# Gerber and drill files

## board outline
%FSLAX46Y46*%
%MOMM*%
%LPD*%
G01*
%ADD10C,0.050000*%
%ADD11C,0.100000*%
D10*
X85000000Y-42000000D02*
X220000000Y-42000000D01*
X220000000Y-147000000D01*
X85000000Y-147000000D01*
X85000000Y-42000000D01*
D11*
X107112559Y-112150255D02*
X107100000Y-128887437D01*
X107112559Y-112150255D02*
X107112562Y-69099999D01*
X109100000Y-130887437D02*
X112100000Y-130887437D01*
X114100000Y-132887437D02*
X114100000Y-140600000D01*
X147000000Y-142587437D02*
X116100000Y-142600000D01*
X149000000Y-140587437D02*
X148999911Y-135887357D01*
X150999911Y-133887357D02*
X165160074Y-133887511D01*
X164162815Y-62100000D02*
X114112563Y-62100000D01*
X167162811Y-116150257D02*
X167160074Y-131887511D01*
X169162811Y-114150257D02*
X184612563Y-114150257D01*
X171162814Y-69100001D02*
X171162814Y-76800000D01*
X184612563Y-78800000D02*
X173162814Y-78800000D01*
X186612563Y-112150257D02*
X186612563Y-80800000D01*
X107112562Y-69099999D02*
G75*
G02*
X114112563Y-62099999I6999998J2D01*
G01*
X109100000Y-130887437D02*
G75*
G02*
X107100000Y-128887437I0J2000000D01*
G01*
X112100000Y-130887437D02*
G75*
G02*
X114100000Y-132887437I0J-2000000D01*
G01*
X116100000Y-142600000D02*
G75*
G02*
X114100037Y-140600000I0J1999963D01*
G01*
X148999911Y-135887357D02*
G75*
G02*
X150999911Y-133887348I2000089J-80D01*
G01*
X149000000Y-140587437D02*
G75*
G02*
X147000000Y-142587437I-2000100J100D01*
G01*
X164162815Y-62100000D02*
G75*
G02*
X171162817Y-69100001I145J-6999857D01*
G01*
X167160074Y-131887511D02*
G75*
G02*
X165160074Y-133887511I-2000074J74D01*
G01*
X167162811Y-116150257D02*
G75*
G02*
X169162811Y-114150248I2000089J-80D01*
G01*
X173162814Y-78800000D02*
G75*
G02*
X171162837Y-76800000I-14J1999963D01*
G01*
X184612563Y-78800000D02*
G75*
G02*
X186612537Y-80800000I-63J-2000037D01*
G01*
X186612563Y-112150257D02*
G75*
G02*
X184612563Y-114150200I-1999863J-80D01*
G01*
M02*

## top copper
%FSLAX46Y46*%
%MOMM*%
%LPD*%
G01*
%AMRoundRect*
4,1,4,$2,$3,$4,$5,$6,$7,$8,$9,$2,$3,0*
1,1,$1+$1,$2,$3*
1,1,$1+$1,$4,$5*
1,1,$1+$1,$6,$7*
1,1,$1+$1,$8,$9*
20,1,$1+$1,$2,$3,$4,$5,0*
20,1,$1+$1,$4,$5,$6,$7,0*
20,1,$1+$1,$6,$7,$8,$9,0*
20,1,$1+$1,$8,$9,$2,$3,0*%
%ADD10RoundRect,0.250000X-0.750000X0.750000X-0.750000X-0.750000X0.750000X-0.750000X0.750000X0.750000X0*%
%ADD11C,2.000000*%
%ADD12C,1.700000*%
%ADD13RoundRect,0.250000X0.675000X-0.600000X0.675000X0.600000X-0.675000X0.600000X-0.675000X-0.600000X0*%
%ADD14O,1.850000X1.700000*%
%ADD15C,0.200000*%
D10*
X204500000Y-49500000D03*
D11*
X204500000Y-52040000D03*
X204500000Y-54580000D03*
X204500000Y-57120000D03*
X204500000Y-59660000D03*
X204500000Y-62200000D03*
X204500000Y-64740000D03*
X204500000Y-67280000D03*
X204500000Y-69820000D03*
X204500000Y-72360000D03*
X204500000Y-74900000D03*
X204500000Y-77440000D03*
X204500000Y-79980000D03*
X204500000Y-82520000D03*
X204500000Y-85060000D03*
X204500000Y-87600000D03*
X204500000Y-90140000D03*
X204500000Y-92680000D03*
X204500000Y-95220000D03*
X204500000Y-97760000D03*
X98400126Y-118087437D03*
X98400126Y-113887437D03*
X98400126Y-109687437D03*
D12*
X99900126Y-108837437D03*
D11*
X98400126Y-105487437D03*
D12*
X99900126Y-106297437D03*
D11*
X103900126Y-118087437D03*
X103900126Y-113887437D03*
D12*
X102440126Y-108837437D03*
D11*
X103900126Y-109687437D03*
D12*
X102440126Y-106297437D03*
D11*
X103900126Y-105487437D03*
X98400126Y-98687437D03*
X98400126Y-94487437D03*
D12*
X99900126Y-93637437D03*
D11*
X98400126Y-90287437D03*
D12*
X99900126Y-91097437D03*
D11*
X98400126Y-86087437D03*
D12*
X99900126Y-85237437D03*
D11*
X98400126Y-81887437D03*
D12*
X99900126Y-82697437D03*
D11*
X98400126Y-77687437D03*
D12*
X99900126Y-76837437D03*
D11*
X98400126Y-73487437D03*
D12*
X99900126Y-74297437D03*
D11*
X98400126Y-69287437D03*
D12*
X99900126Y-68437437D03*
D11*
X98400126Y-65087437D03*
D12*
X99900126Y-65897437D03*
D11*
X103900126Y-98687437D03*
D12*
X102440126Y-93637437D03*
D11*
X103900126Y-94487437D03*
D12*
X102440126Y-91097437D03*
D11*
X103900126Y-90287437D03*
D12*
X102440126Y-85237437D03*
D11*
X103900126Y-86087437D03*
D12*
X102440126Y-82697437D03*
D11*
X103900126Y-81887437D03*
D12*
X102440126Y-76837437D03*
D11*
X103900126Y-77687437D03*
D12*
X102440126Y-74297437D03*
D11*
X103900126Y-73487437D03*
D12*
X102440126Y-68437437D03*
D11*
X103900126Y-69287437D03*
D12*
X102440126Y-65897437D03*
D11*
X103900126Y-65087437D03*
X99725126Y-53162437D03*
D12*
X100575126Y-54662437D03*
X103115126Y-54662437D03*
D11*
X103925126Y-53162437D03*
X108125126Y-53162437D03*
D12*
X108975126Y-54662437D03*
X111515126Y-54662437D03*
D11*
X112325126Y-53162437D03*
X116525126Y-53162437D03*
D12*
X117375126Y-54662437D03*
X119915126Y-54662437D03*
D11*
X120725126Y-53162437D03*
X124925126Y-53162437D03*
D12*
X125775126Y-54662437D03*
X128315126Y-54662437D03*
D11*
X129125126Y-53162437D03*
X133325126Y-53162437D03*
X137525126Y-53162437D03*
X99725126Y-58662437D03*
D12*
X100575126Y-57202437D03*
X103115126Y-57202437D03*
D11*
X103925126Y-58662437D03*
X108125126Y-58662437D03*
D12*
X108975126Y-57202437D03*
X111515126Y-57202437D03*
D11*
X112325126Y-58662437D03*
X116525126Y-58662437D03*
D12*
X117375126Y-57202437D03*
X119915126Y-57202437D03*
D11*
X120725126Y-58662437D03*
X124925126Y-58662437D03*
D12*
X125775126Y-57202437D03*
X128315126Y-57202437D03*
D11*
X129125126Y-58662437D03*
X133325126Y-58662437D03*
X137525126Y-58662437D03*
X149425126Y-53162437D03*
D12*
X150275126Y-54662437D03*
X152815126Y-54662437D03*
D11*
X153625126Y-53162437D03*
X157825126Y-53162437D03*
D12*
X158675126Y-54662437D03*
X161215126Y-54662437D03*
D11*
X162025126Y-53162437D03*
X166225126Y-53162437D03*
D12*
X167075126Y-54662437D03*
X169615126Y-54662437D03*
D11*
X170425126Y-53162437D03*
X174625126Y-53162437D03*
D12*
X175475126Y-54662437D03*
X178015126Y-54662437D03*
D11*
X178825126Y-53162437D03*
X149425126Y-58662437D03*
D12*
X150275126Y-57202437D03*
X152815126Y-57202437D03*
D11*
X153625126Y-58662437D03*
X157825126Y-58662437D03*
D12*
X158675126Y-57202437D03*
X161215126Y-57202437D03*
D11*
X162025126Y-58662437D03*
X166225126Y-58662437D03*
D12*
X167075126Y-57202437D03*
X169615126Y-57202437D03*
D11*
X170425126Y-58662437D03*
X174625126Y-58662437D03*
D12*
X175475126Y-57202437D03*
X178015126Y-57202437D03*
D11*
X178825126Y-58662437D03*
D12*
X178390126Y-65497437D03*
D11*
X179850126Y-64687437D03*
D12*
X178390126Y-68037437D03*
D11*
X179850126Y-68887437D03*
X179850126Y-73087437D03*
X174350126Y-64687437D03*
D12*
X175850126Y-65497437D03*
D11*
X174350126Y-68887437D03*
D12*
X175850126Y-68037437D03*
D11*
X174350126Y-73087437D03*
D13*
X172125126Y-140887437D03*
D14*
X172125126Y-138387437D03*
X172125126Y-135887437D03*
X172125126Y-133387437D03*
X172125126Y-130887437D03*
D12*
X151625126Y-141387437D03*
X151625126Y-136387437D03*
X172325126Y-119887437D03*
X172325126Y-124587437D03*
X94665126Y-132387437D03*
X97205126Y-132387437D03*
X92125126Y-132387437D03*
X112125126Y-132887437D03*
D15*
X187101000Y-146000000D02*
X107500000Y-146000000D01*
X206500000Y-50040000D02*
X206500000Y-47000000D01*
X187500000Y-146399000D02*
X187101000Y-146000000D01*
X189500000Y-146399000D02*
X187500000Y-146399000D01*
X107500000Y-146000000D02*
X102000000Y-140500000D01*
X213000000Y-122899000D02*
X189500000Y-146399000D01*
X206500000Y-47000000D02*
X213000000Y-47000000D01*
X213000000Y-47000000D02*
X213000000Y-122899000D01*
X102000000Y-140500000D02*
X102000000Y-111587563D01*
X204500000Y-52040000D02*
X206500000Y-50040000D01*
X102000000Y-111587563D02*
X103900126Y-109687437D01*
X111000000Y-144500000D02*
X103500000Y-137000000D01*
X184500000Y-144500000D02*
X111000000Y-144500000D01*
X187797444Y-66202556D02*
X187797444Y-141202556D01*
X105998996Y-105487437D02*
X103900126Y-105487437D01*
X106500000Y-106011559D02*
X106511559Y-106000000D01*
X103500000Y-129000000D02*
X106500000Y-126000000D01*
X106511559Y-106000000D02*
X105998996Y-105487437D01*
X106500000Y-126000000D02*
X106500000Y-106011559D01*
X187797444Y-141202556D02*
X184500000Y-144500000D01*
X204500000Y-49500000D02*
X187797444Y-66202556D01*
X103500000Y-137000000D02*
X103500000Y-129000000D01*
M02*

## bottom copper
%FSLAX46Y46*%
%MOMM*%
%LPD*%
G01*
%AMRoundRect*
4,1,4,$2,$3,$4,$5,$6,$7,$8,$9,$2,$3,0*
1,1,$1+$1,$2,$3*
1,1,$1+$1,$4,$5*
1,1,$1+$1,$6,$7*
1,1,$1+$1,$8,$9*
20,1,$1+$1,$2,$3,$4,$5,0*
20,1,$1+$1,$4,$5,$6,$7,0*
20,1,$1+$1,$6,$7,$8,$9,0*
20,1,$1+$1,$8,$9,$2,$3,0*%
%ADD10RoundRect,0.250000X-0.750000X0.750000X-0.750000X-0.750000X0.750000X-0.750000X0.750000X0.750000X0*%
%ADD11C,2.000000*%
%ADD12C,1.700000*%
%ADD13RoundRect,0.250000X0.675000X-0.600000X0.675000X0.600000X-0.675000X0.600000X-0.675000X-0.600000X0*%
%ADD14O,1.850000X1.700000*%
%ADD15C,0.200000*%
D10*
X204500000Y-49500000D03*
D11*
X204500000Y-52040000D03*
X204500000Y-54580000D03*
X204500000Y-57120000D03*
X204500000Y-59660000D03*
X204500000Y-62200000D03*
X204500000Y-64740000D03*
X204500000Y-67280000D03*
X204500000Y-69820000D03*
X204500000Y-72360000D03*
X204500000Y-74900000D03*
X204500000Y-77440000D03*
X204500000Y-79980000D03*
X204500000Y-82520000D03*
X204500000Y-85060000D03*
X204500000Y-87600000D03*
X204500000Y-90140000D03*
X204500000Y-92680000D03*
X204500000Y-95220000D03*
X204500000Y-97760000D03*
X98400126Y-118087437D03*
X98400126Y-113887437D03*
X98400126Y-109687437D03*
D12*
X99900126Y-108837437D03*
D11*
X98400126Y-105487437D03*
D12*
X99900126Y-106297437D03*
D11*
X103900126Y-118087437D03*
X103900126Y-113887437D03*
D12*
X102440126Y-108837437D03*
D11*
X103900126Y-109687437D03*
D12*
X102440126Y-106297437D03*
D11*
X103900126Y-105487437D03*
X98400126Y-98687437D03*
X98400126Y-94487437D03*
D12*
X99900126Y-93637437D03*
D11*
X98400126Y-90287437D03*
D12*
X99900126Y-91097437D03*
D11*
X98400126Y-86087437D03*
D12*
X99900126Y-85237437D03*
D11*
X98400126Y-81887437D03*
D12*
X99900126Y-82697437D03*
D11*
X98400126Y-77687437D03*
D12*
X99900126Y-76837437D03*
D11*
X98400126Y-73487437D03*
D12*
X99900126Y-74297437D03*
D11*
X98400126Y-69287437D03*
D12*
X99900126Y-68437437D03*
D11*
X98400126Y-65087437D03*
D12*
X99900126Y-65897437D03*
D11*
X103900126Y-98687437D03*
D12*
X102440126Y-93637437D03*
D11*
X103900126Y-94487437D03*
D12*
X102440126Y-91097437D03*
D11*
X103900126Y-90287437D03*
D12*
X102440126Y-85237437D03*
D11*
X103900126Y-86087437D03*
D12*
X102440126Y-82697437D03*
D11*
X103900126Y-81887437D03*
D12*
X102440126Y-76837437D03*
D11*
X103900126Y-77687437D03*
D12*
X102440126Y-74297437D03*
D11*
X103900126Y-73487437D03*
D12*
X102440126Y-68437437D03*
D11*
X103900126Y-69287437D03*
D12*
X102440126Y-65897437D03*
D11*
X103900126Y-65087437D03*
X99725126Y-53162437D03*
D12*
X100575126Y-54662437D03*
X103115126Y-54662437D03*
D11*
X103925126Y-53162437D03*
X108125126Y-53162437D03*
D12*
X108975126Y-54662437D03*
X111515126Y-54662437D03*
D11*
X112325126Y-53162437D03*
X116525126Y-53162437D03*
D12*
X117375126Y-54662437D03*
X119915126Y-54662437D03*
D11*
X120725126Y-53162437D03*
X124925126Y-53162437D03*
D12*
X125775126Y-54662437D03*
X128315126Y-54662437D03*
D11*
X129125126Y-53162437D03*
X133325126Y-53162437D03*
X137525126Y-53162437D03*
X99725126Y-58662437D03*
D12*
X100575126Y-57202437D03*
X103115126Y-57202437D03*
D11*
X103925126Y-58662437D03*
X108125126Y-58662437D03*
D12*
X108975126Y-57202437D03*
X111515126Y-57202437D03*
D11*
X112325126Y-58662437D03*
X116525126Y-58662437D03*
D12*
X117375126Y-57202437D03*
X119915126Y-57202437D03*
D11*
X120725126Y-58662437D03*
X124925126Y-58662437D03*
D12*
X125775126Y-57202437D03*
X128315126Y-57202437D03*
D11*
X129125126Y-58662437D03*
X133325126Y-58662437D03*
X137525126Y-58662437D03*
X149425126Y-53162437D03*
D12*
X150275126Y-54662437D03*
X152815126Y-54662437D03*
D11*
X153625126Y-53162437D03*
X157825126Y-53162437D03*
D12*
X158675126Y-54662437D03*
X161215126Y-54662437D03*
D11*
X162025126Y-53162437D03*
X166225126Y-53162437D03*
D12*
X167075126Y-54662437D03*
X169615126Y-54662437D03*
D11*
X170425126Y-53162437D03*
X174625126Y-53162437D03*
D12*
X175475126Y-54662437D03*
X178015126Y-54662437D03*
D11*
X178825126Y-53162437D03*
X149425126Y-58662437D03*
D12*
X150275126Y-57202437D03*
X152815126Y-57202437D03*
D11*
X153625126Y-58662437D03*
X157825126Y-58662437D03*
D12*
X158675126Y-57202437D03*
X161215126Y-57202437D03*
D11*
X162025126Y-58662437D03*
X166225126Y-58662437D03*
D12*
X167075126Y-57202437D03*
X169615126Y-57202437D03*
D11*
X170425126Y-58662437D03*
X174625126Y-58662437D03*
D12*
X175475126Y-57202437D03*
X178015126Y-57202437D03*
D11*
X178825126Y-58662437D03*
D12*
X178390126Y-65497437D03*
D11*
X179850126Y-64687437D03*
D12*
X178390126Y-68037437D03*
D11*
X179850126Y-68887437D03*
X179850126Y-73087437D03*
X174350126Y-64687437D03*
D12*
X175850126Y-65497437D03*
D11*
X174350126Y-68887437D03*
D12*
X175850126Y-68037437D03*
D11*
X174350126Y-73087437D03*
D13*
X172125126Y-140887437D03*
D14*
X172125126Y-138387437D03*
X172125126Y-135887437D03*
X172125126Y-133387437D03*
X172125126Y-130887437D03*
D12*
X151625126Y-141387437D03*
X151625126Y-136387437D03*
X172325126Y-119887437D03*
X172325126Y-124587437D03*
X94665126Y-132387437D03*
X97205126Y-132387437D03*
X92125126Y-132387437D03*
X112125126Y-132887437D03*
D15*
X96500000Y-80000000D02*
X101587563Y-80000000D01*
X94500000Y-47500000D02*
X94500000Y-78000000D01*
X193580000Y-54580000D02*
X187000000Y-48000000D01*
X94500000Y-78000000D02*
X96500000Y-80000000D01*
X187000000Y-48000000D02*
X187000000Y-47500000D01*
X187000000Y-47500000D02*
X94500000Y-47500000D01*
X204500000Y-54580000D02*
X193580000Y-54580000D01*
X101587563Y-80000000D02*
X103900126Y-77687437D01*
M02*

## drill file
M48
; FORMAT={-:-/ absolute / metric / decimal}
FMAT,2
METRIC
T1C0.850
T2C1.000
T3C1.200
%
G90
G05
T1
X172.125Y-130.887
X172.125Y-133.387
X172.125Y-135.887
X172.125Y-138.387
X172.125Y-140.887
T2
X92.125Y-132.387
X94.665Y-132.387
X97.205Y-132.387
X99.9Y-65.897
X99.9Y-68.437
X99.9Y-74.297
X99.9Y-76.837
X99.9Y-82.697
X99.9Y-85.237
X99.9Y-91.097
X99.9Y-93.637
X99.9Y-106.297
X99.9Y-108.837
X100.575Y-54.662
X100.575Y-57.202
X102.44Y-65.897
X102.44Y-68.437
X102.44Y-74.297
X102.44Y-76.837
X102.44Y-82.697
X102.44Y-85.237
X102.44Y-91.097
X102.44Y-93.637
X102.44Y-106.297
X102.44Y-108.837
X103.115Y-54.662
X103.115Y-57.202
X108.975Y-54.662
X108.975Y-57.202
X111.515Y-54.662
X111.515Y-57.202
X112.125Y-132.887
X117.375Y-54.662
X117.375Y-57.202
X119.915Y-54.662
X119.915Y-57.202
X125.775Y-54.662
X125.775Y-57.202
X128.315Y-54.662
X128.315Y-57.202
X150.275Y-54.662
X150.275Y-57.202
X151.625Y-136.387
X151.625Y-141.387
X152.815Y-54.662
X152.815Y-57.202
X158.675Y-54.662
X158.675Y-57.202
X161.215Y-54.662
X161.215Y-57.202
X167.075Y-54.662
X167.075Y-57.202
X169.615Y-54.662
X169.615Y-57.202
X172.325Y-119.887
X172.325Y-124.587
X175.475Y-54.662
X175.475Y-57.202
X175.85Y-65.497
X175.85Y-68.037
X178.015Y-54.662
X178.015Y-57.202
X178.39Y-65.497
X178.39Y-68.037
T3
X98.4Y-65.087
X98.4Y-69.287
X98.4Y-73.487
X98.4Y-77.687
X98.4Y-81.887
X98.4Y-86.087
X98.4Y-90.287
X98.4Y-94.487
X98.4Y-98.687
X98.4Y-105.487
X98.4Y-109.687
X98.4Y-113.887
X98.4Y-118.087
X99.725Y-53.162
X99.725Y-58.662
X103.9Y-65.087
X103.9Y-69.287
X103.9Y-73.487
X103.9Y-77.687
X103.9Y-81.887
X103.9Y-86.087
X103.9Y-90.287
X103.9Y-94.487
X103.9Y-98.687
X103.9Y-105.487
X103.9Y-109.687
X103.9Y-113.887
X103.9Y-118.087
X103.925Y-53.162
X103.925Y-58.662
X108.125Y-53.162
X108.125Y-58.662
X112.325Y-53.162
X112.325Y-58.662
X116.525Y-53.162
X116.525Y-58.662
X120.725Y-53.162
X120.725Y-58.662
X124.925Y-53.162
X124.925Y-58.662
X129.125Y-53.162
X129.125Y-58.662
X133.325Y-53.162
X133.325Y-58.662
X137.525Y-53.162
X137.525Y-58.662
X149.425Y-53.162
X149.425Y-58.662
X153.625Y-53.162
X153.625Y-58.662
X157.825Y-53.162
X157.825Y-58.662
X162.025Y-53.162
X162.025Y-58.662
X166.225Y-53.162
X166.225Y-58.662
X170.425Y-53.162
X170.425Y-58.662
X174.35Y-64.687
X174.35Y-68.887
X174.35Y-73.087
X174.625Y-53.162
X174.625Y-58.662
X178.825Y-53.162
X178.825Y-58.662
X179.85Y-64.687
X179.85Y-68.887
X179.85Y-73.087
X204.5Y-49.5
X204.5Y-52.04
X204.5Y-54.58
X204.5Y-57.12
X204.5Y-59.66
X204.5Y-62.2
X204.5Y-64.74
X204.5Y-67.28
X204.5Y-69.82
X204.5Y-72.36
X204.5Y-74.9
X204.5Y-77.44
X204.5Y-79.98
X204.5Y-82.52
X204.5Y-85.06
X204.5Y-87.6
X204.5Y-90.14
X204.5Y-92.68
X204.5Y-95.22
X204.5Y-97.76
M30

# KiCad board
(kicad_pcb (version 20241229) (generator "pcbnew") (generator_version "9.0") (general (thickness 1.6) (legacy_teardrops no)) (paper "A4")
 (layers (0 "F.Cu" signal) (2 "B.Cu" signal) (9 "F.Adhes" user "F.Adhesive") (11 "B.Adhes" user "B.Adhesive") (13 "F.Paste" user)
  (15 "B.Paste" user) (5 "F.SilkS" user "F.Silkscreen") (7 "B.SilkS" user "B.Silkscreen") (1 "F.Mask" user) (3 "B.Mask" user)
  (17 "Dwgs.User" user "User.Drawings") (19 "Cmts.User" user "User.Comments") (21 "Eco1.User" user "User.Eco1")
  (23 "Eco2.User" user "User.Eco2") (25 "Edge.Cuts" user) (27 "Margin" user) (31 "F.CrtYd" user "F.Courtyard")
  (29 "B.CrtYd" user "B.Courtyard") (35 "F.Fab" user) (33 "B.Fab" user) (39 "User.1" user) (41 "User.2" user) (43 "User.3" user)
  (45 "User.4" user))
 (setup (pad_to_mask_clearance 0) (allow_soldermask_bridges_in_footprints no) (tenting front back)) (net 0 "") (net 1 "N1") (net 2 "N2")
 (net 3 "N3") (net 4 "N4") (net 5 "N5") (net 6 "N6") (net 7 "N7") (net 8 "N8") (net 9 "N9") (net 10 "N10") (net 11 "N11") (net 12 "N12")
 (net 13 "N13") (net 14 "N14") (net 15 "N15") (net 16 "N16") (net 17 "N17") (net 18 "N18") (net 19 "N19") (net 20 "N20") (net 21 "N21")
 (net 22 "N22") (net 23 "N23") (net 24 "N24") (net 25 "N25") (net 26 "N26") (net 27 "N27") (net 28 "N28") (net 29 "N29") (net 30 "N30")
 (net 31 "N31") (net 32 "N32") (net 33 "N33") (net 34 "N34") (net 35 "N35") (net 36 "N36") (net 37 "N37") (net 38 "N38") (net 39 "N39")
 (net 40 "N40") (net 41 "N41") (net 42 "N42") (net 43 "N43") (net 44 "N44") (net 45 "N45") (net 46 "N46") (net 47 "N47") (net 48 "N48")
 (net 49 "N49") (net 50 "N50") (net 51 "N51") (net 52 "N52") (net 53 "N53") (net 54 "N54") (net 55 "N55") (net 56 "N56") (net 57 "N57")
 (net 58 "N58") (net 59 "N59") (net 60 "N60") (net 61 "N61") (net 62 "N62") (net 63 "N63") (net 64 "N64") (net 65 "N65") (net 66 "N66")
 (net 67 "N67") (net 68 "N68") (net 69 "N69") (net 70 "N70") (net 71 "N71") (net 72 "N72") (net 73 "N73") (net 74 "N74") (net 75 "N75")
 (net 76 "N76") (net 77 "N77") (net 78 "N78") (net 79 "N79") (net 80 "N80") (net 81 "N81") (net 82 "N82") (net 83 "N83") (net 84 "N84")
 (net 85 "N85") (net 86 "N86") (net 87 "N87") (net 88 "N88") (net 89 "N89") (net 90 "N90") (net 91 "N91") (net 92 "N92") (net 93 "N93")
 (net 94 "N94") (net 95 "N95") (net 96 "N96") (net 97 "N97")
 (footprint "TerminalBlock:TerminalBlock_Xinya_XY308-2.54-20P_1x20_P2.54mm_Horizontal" (layer "F.Cu") (at 204.5 49.5 -90)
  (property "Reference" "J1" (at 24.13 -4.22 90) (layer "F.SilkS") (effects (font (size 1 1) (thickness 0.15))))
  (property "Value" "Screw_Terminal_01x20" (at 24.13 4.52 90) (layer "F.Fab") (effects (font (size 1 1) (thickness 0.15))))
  (pad "1" thru_hole roundrect (at 0 0 270) (size 2 2) (drill 1.2) (layers "*.Cu" "*.Mask") (remove_unused_layers no)
   (roundrect_rratio 0.125) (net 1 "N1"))
  (pad "2" thru_hole circle (at 2.54 0 270) (size 2 2) (drill 1.2) (layers "*.Cu" "*.Mask") (remove_unused_layers no) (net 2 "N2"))
  (pad "3" thru_hole circle (at 5.08 0 270) (size 2 2) (drill 1.2) (layers "*.Cu" "*.Mask") (remove_unused_layers no) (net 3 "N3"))
  (pad "4" thru_hole circle (at 7.62 0 270) (size 2 2) (drill 1.2) (layers "*.Cu" "*.Mask") (remove_unused_layers no) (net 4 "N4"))
  (pad "5" thru_hole circle (at 10.16 0 270) (size 2 2) (drill 1.2) (layers "*.Cu" "*.Mask") (remove_unused_layers no) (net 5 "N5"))
  (pad "6" thru_hole circle (at 12.7 0 270) (size 2 2) (drill 1.2) (layers "*.Cu" "*.Mask") (remove_unused_layers no) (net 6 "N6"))
  (pad "7" thru_hole circle (at 15.24 0 270) (size 2 2) (drill 1.2) (layers "*.Cu" "*.Mask") (remove_unused_layers no) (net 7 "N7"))
  (pad "8" thru_hole circle (at 17.78 0 270) (size 2 2) (drill 1.2) (layers "*.Cu" "*.Mask") (remove_unused_layers no) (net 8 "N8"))
  (pad "9" thru_hole circle (at 20.32 0 270) (size 2 2) (drill 1.2) (layers "*.Cu" "*.Mask") (remove_unused_layers no) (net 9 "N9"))
  (pad "10" thru_hole circle (at 22.86 0 270) (size 2 2) (drill 1.2) (layers "*.Cu" "*.Mask") (remove_unused_layers no) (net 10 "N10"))
  (pad "11" thru_hole circle (at 25.4 0 270) (size 2 2) (drill 1.2) (layers "*.Cu" "*.Mask") (remove_unused_layers no) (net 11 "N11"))
  (pad "12" thru_hole circle (at 27.94 0 270) (size 2 2) (drill 1.2) (layers "*.Cu" "*.Mask") (remove_unused_layers no) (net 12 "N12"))
  (pad "13" thru_hole circle (at 30.48 0 270) (size 2 2) (drill 1.2) (layers "*.Cu" "*.Mask") (remove_unused_layers no) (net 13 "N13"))
  (pad "14" thru_hole circle (at 33.02 0 270) (size 2 2) (drill 1.2) (layers "*.Cu" "*.Mask") (remove_unused_layers no) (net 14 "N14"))
  (pad "15" thru_hole circle (at 35.56 0 270) (size 2 2) (drill 1.2) (layers "*.Cu" "*.Mask") (remove_unused_layers no) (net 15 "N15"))
  (pad "16" thru_hole circle (at 38.1 0 270) (size 2 2) (drill 1.2) (layers "*.Cu" "*.Mask") (remove_unused_layers no) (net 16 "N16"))
  (pad "17" thru_hole circle (at 40.64 0 270) (size 2 2) (drill 1.2) (layers "*.Cu" "*.Mask") (remove_unused_layers no) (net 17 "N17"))
  (pad "18" thru_hole circle (at 43.18 0 270) (size 2 2) (drill 1.2) (layers "*.Cu" "*.Mask") (remove_unused_layers no) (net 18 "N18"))
  (pad "19" thru_hole circle (at 45.72 0 270) (size 2 2) (drill 1.2) (layers "*.Cu" "*.Mask") (remove_unused_layers no) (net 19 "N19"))
  (pad "20" thru_hole circle (at 48.26 0 270) (size 2 2) (drill 1.2) (layers "*.Cu" "*.Mask") (remove_unused_layers no) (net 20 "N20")))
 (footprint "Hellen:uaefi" (layer "F.Cu") (at 89.1 143.887437)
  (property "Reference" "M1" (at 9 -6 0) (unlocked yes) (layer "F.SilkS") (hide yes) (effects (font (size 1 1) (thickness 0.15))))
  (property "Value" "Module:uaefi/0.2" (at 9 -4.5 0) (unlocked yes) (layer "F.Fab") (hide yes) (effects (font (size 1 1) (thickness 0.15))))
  (fp_line (start 18.012559 -31.737182) (end 18 -15) (stroke (width 0.1) (type default)) (layer "Edge.Cuts"))
  (fp_line (start 18.012559 -31.737182) (end 18.012562 -74.787438) (stroke (width 0.1) (type default)) (layer "Edge.Cuts"))
  (fp_line (start 20 -13) (end 23 -13) (stroke (width 0.1) (type default)) (layer "Edge.Cuts"))
  (fp_line (start 25 -11) (end 25 -3.287437) (stroke (width 0.1) (type default)) (layer "Edge.Cuts"))
  (fp_line (start 57.9 -1.3) (end 27 -1.287437) (stroke (width 0.1) (type default)) (layer "Edge.Cuts"))
  (fp_line (start 59.9 -3.3) (end 59.899911 -8.00008) (stroke (width 0.1) (type default)) (layer "Edge.Cuts"))
  (fp_line (start 61.899911 -10.00008) (end 76.060074 -9.999926) (stroke (width 0.1) (type default)) (layer "Edge.Cuts"))
  (fp_line (start 75.062815 -81.787437) (end 25.012563 -81.787437) (stroke (width 0.1) (type default)) (layer "Edge.Cuts"))
  (fp_line (start 78.062811 -27.73718) (end 78.060074 -11.999926) (stroke (width 0.1) (type default)) (layer "Edge.Cuts"))
  (fp_line (start 80.062811 -29.73718) (end 95.512563 -29.73718) (stroke (width 0.1) (type default)) (layer "Edge.Cuts"))
  (fp_line (start 82.062814 -74.787436) (end 82.062814 -67.087437) (stroke (width 0.1) (type default)) (layer "Edge.Cuts"))
  (fp_line (start 95.512563 -65.087437) (end 84.062814 -65.087437) (stroke (width 0.1) (type default)) (layer "Edge.Cuts"))
  (fp_line (start 97.512563 -31.73718) (end 97.512563 -63.087437) (stroke (width 0.1) (type default)) (layer "Edge.Cuts"))
  (fp_arc (start 18.012562 -74.787438) (mid 20.062815 -79.737185) (end 25.012563 -81.787437) (stroke (width 0.1) (type solid))
   (layer "Edge.Cuts"))
  (fp_arc (start 20 -13) (mid 18.585784 -13.585784) (end 18 -15) (stroke (width 0.1) (type default)) (layer "Edge.Cuts"))
  (fp_arc (start 23 -13) (mid 24.414216 -12.414216) (end 25 -11) (stroke (width 0.1) (type default)) (layer "Edge.Cuts"))
  (fp_arc (start 27 -1.287437) (mid 25.585783 -1.873222) (end 25 -3.287437) (stroke (width 0.1) (type default)) (layer "Edge.Cuts"))
  (fp_arc (start 59.899911 -8.00008) (mid 60.485719 -9.414272) (end 61.899911 -10.00008) (stroke (width 0.1) (type default))
   (layer "Edge.Cuts"))
  (fp_arc (start 59.9 -3.3) (mid 59.314192 -1.885808) (end 57.9 -1.3) (stroke (width 0.1) (type default)) (layer "Edge.Cuts"))
  (fp_arc (start 75.062815 -81.787437) (mid 80.012612 -79.73722) (end 82.062814 -74.787436) (stroke (width 0.1) (type solid))
   (layer "Edge.Cuts"))
  (fp_arc (start 78.060074 -11.999926) (mid 77.474266 -10.585734) (end 76.060074 -9.999926) (stroke (width 0.1) (type default))
   (layer "Edge.Cuts"))
  (fp_arc (start 78.062811 -27.73718) (mid 78.648619 -29.151383) (end 80.062811 -29.73718) (stroke (width 0.1) (type default))
   (layer "Edge.Cuts"))
  (fp_arc (start 84.062814 -65.087437) (mid 82.648592 -65.673201) (end 82.062814 -67.087437) (stroke (width 0.1) (type default))
   (layer "Edge.Cuts"))
  (fp_arc (start 95.512563 -65.087437) (mid 96.926766 -64.50164) (end 97.512563 -63.087437) (stroke (width 0.1) (type default))
   (layer "Edge.Cuts"))
  (fp_arc (start 97.512563 -31.73718) (mid 96.926801 -30.322937) (end 95.512563 -29.73718) (stroke (width 0.1) (type default))
   (layer "Edge.Cuts"))
  (pad "A1" thru_hole circle (at 9.300126 -25.8 90) (size 2 2) (drill 1.2) (layers "*.Cu" "*.Mask") (remove_unused_layers no) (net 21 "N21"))
  (pad "A2" thru_hole circle (at 9.300126 -30 90) (size 2 2) (drill 1.2) (layers "*.Cu" "*.Mask") (remove_unused_layers no) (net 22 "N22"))
  (pad "A3" thru_hole circle (at 9.300126 -34.2 90) (size 2 2) (drill 1.2) (layers "*.Cu" "*.Mask") (remove_unused_layers no) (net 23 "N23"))
  (pad "A3" thru_hole circle (at 10.800126 -35.05 180) (size 1.7 1.7) (drill 1) (layers "*.Cu" "*.Mask") (remove_unused_layers no)
   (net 23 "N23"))
  (pad "A4" thru_hole circle (at 9.300126 -38.4 90) (size 2 2) (drill 1.2) (layers "*.Cu" "*.Mask") (remove_unused_layers no) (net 3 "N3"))
  (pad "A4" thru_hole circle (at 10.800126 -37.59 180) (size 1.7 1.7) (drill 1) (layers "*.Cu" "*.Mask") (remove_unused_layers no)
   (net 3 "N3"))
  (pad "A5" thru_hole circle (at 14.800126 -25.8 90) (size 2 2) (drill 1.2) (layers "*.Cu" "*.Mask") (remove_unused_layers no)
   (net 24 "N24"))
  (pad "A6" thru_hole circle (at 14.800126 -30 90) (size 2 2) (drill 1.2) (layers "*.Cu" "*.Mask") (remove_unused_layers no) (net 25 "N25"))
  (pad "A7" thru_hole circle (at 13.340126 -35.05 180) (size 1.7 1.7) (drill 1) (layers "*.Cu" "*.Mask") (remove_unused_layers no)
   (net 2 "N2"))
  (pad "A7" thru_hole circle (at 14.800126 -34.2 90) (size 2 2) (drill 1.2) (layers "*.Cu" "*.Mask") (remove_unused_layers no) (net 2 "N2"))
  (pad "A8" thru_hole circle (at 13.340126 -37.59 180) (size 1.7 1.7) (drill 1) (layers "*.Cu" "*.Mask") (remove_unused_layers no)
   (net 1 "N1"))
  (pad "A8" thru_hole circle (at 14.800126 -38.4 90) (size 2 2) (drill 1.2) (layers "*.Cu" "*.Mask") (remove_unused_layers no) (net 1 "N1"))
  (pad "B1" thru_hole circle (at 9.300126 -45.2 90) (size 2 2) (drill 1.2) (layers "*.Cu" "*.Mask") (remove_unused_layers no) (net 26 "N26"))
  (pad "B2" thru_hole circle (at 9.300126 -49.4 90) (size 2 2) (drill 1.2) (layers "*.Cu" "*.Mask") (remove_unused_layers no) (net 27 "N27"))
  (pad "B2" thru_hole circle (at 10.800126 -50.25 180) (size 1.7 1.7) (drill 1) (layers "*.Cu" "*.Mask") (remove_unused_layers no)
   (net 27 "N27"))
  (pad "B3" thru_hole circle (at 9.300126 -53.6 90) (size 2 2) (drill 1.2) (layers "*.Cu" "*.Mask") (remove_unused_layers no) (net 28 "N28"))
  (pad "B3" thru_hole circle (at 10.800126 -52.79 180) (size 1.7 1.7) (drill 1) (layers "*.Cu" "*.Mask") (remove_unused_layers no)
   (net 28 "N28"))
  (pad "B4" thru_hole circle (at 9.300126 -57.8 90) (size 2 2) (drill 1.2) (layers "*.Cu" "*.Mask") (remove_unused_layers no) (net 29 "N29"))
  (pad "B4" thru_hole circle (at 10.800126 -58.65 180) (size 1.7 1.7) (drill 1) (layers "*.Cu" "*.Mask") (remove_unused_layers no)
   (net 29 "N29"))
  (pad "B5" thru_hole circle (at 9.300126 -62 90) (size 2 2) (drill 1.2) (layers "*.Cu" "*.Mask") (remove_unused_layers no) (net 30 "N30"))
  (pad "B5" thru_hole circle (at 10.800126 -61.19 180) (size 1.7 1.7) (drill 1) (layers "*.Cu" "*.Mask") (remove_unused_layers no)
   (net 30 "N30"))
  (pad "B6" thru_hole circle (at 9.300126 -66.2 90) (size 2 2) (drill 1.2) (layers "*.Cu" "*.Mask") (remove_unused_layers no) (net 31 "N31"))
  (pad "B6" thru_hole circle (at 10.800126 -67.05 180) (size 1.7 1.7) (drill 1) (layers "*.Cu" "*.Mask") (remove_unused_layers no)
   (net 31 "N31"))
  (pad "B7" thru_hole circle (at 9.300126 -70.4 90) (size 2 2) (drill 1.2) (layers "*.Cu" "*.Mask") (remove_unused_layers no) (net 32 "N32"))
  (pad "B7" thru_hole circle (at 10.800126 -69.59 180) (size 1.7 1.7) (drill 1) (layers "*.Cu" "*.Mask") (remove_unused_layers no)
   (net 32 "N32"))
  (pad "B8" thru_hole circle (at 9.300126 -74.6 90) (size 2 2) (drill 1.2) (layers "*.Cu" "*.Mask") (remove_unused_layers no) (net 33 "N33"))
  (pad "B8" thru_hole circle (at 10.800126 -75.45 180) (size 1.7 1.7) (drill 1) (layers "*.Cu" "*.Mask") (remove_unused_layers no)
   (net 33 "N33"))
  (pad "B9" thru_hole circle (at 9.300126 -78.8 90) (size 2 2) (drill 1.2) (layers "*.Cu" "*.Mask") (remove_unused_layers no) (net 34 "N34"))
  (pad "B9" thru_hole circle (at 10.800126 -77.99 180) (size 1.7 1.7) (drill 1) (layers "*.Cu" "*.Mask") (remove_unused_layers no)
   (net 34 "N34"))
  (pad "B10" thru_hole circle (at 14.800126 -45.2 90) (size 2 2) (drill 1.2) (layers "*.Cu" "*.Mask") (remove_unused_layers no)
   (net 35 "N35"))
  (pad "B11" thru_hole circle (at 13.340126 -50.25 180) (size 1.7 1.7) (drill 1) (layers "*.Cu" "*.Mask") (remove_unused_layers no)
   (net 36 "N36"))
  (pad "B11" thru_hole circle (at 14.800126 -49.4 90) (size 2 2) (drill 1.2) (layers "*.Cu" "*.Mask") (remove_unused_layers no)
   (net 36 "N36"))
  (pad "B12" thru_hole circle (at 13.340126 -52.79 180) (size 1.7 1.7) (drill 1) (layers "*.Cu" "*.Mask") (remove_unused_layers no)
   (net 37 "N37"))
  (pad "B12" thru_hole circle (at 14.800126 -53.6 90) (size 2 2) (drill 1.2) (layers "*.Cu" "*.Mask") (remove_unused_layers no)
   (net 37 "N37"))
  (pad "B13" thru_hole circle (at 13.340126 -58.65 180) (size 1.7 1.7) (drill 1) (layers "*.Cu" "*.Mask") (remove_unused_layers no)
   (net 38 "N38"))
  (pad "B13" thru_hole circle (at 14.800126 -57.8 90) (size 2 2) (drill 1.2) (layers "*.Cu" "*.Mask") (remove_unused_layers no)
   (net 38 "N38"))
  (pad "B14" thru_hole circle (at 13.340126 -61.19 180) (size 1.7 1.7) (drill 1) (layers "*.Cu" "*.Mask") (remove_unused_layers no)
   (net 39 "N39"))
  (pad "B14" thru_hole circle (at 14.800126 -62 90) (size 2 2) (drill 1.2) (layers "*.Cu" "*.Mask") (remove_unused_layers no) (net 39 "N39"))
  (pad "B15" thru_hole circle (at 13.340126 -67.05 180) (size 1.7 1.7) (drill 1) (layers "*.Cu" "*.Mask") (remove_unused_layers no)
   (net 3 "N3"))
  (pad "B15" thru_hole circle (at 14.800126 -66.2 90) (size 2 2) (drill 1.2) (layers "*.Cu" "*.Mask") (remove_unused_layers no) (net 3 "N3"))
  (pad "B16" thru_hole circle (at 13.340126 -69.59 180) (size 1.7 1.7) (drill 1) (layers "*.Cu" "*.Mask") (remove_unused_layers no)
   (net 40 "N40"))
  (pad "B16" thru_hole circle (at 14.800126 -70.4 90) (size 2 2) (drill 1.2) (layers "*.Cu" "*.Mask") (remove_unused_layers no)
   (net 40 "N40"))
  (pad "B17" thru_hole circle (at 13.340126 -75.45 180) (size 1.7 1.7) (drill 1) (layers "*.Cu" "*.Mask") (remove_unused_layers no)
   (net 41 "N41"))
  (pad "B17" thru_hole circle (at 14.800126 -74.6 90) (size 2 2) (drill 1.2) (layers "*.Cu" "*.Mask") (remove_unused_layers no)
   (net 41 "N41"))
  (pad "B18" thru_hole circle (at 13.340126 -77.99 180) (size 1.7 1.7) (drill 1) (layers "*.Cu" "*.Mask") (remove_unused_layers no)
   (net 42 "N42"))
  (pad "B18" thru_hole circle (at 14.800126 -78.8 90) (size 2 2) (drill 1.2) (layers "*.Cu" "*.Mask") (remove_unused_layers no)
   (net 42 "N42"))
  (pad "C1" thru_hole circle (at 10.625126 -90.725 90) (size 2 2) (drill 1.2) (layers "*.Cu" "*.Mask") (remove_unused_layers no)
   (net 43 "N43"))
  (pad "C1" thru_hole circle (at 11.475126 -89.225 90) (size 1.7 1.7) (drill 1) (layers "*.Cu" "*.Mask") (remove_unused_layers no)
   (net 43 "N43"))
  (pad "C2" thru_hole circle (at 14.015126 -89.225 90) (size 1.7 1.7) (drill 1) (layers "*.Cu" "*.Mask") (remove_unused_layers no)
   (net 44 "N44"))
  (pad "C2" thru_hole circle (at 14.825126 -90.725 90) (size 2 2) (drill 1.2) (layers "*.Cu" "*.Mask") (remove_unused_layers no)
   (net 44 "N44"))
  (pad "C3" thru_hole circle (at 19.025126 -90.725 90) (size 2 2) (drill 1.2) (layers "*.Cu" "*.Mask") (remove_unused_layers no)
   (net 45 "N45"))
  (pad "C3" thru_hole circle (at 19.875126 -89.225 90) (size 1.7 1.7) (drill 1) (layers "*.Cu" "*.Mask") (remove_unused_layers no)
   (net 45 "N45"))
  (pad "C4" thru_hole circle (at 22.415126 -89.225 90) (size 1.7 1.7) (drill 1) (layers "*.Cu" "*.Mask") (remove_unused_layers no)
   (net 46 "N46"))
  (pad "C4" thru_hole circle (at 23.225126 -90.725 90) (size 2 2) (drill 1.2) (layers "*.Cu" "*.Mask") (remove_unused_layers no)
   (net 46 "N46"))
  (pad "C5" thru_hole circle (at 27.425126 -90.725 90) (size 2 2) (drill 1.2) (layers "*.Cu" "*.Mask") (remove_unused_layers no)
   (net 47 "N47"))
  (pad "C5" thru_hole circle (at 28.275126 -89.225 90) (size 1.7 1.7) (drill 1) (layers "*.Cu" "*.Mask") (remove_unused_layers no)
   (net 47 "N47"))
  (pad "C6" thru_hole circle (at 30.815126 -89.225 90) (size 1.7 1.7) (drill 1) (layers "*.Cu" "*.Mask") (remove_unused_layers no)
   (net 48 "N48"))
  (pad "C6" thru_hole circle (at 31.625126 -90.725 90) (size 2 2) (drill 1.2) (layers "*.Cu" "*.Mask") (remove_unused_layers no)
   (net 48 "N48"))
  (pad "C7" thru_hole circle (at 35.825126 -90.725 90) (size 2 2) (drill 1.2) (layers "*.Cu" "*.Mask") (remove_unused_layers no)
   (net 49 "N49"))
  (pad "C7" thru_hole circle (at 36.675126 -89.225 90) (size 1.7 1.7) (drill 1) (layers "*.Cu" "*.Mask") (remove_unused_layers no)
   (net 49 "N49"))
  (pad "C8" thru_hole circle (at 39.215126 -89.225 90) (size 1.7 1.7) (drill 1) (layers "*.Cu" "*.Mask") (remove_unused_layers no)
   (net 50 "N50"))
  (pad "C8" thru_hole circle (at 40.025126 -90.725 90) (size 2 2) (drill 1.2) (layers "*.Cu" "*.Mask") (remove_unused_layers no)
   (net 50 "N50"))
  (pad "C9" thru_hole circle (at 44.225126 -90.725 90) (size 2 2) (drill 1.2) (layers "*.Cu" "*.Mask") (remove_unused_layers no)
   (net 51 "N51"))
  (pad "C10" thru_hole circle (at 48.425126 -90.725 90) (size 2 2) (drill 1.2) (layers "*.Cu" "*.Mask") (remove_unused_layers no)
   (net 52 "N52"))
  (pad "C11" thru_hole circle (at 10.625126 -85.225 90) (size 2 2) (drill 1.2) (layers "*.Cu" "*.Mask") (remove_unused_layers no)
   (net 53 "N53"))
  (pad "C11" thru_hole circle (at 11.475126 -86.685 90) (size 1.7 1.7) (drill 1) (layers "*.Cu" "*.Mask") (remove_unused_layers no)
   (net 53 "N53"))
  (pad "C12" thru_hole circle (at 14.015126 -86.685 90) (size 1.7 1.7) (drill 1) (layers "*.Cu" "*.Mask") (remove_unused_layers no)
   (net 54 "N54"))
  (pad "C12" thru_hole circle (at 14.825126 -85.225 90) (size 2 2) (drill 1.2) (layers "*.Cu" "*.Mask") (remove_unused_layers no)
   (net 54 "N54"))
  (pad "C13" thru_hole circle (at 19.025126 -85.225 90) (size 2 2) (drill 1.2) (layers "*.Cu" "*.Mask") (remove_unused_layers no)
   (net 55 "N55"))
  (pad "C13" thru_hole circle (at 19.875126 -86.685 90) (size 1.7 1.7) (drill 1) (layers "*.Cu" "*.Mask") (remove_unused_layers no)
   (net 55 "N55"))
  (pad "C14" thru_hole circle (at 22.415126 -86.685 90) (size 1.7 1.7) (drill 1) (layers "*.Cu" "*.Mask") (remove_unused_layers no)
   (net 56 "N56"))
  (pad "C14" thru_hole circle (at 23.225126 -85.225 90) (size 2 2) (drill 1.2) (layers "*.Cu" "*.Mask") (remove_unused_layers no)
   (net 56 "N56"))
  (pad "C15" thru_hole circle (at 27.425126 -85.225 90) (size 2 2) (drill 1.2) (layers "*.Cu" "*.Mask") (remove_unused_layers no)
   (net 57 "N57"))
  (pad "C15" thru_hole circle (at 28.275126 -86.685 90) (size 1.7 1.7) (drill 1) (layers "*.Cu" "*.Mask") (remove_unused_layers no)
   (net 57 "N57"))
  (pad "C16" thru_hole circle (at 30.815126 -86.685 90) (size 1.7 1.7) (drill 1) (layers "*.Cu" "*.Mask") (remove_unused_layers no)
   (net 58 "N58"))
  (pad "C16" thru_hole circle (at 31.625126 -85.225 90) (size 2 2) (drill 1.2) (layers "*.Cu" "*.Mask") (remove_unused_layers no)
   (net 58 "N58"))
  (pad "C17" thru_hole circle (at 35.825126 -85.225 90) (size 2 2) (drill 1.2) (layers "*.Cu" "*.Mask") (remove_unused_layers no)
   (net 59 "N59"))
  (pad "C17" thru_hole circle (at 36.675126 -86.685 90) (size 1.7 1.7) (drill 1) (layers "*.Cu" "*.Mask") (remove_unused_layers no)
   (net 59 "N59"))
  (pad "C18" thru_hole circle (at 39.215126 -86.685 90) (size 1.7 1.7) (drill 1) (layers "*.Cu" "*.Mask") (remove_unused_layers no)
   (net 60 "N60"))
  (pad "C18" thru_hole circle (at 40.025126 -85.225 90) (size 2 2) (drill 1.2) (layers "*.Cu" "*.Mask") (remove_unused_layers no)
   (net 60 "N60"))
  (pad "C19" thru_hole circle (at 44.225126 -85.225 90) (size 2 2) (drill 1.2) (layers "*.Cu" "*.Mask") (remove_unused_layers no)
   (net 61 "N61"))
  (pad "C20" thru_hole circle (at 48.425126 -85.225 90) (size 2 2) (drill 1.2) (layers "*.Cu" "*.Mask") (remove_unused_layers no)
   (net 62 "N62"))
  (pad "D1" thru_hole circle (at 60.325126 -90.725 90) (size 2 2) (drill 1.2) (layers "*.Cu" "*.Mask") (remove_unused_layers no)
   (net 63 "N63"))
  (pad "D1" thru_hole circle (at 61.175126 -89.225 90) (size 1.7 1.7) (drill 1) (layers "*.Cu" "*.Mask") (remove_unused_layers no)
   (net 63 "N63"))
  (pad "D2" thru_hole circle (at 63.715126 -89.225 90) (size 1.7 1.7) (drill 1) (layers "*.Cu" "*.Mask") (remove_unused_layers no)
   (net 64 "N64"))
  (pad "D2" thru_hole circle (at 64.525126 -90.725 90) (size 2 2) (drill 1.2) (layers "*.Cu" "*.Mask") (remove_unused_layers no)
   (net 64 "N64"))
  (pad "D3" thru_hole circle (at 68.725126 -90.725 90) (size 2 2) (drill 1.2) (layers "*.Cu" "*.Mask") (remove_unused_layers no)
   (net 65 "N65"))
  (pad "D3" thru_hole circle (at 69.575126 -89.225 90) (size 1.7 1.7) (drill 1) (layers "*.Cu" "*.Mask") (remove_unused_layers no)
   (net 65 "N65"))
  (pad "D4" thru_hole circle (at 72.115126 -89.225 90) (size 1.7 1.7) (drill 1) (layers "*.Cu" "*.Mask") (remove_unused_layers no)
   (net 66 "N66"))
  (pad "D4" thru_hole circle (at 72.925126 -90.725 90) (size 2 2) (drill 1.2) (layers "*.Cu" "*.Mask") (remove_unused_layers no)
   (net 66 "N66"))
  (pad "D5" thru_hole circle (at 77.125126 -90.725 90) (size 2 2) (drill 1.2) (layers "*.Cu" "*.Mask") (remove_unused_layers no)
   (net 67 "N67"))
  (pad "D5" thru_hole circle (at 77.975126 -89.225 90) (size 1.7 1.7) (drill 1) (layers "*.Cu" "*.Mask") (remove_unused_layers no)
   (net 67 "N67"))
  (pad "D6" thru_hole circle (at 80.515126 -89.225 90) (size 1.7 1.7) (drill 1) (layers "*.Cu" "*.Mask") (remove_unused_layers no)
   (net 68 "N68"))
  (pad "D6" thru_hole circle (at 81.325126 -90.725 90) (size 2 2) (drill 1.2) (layers "*.Cu" "*.Mask") (remove_unused_layers no)
   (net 68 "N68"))
  (pad "D7" thru_hole circle (at 85.525126 -90.725 90) (size 2 2) (drill 1.2) (layers "*.Cu" "*.Mask") (remove_unused_layers no)
   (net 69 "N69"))
  (pad "D7" thru_hole circle (at 86.375126 -89.225 90) (size 1.7 1.7) (drill 1) (layers "*.Cu" "*.Mask") (remove_unused_layers no)
   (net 69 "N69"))
  (pad "D8" thru_hole circle (at 88.915126 -89.225 90) (size 1.7 1.7) (drill 1) (layers "*.Cu" "*.Mask") (remove_unused_layers no)
   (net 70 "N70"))
  (pad "D8" thru_hole circle (at 89.725126 -90.725 90) (size 2 2) (drill 1.2) (layers "*.Cu" "*.Mask") (remove_unused_layers no)
   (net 70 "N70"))
  (pad "D9" thru_hole circle (at 60.325126 -85.225 90) (size 2 2) (drill 1.2) (layers "*.Cu" "*.Mask") (remove_unused_layers no)
   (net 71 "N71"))
  (pad "D9" thru_hole circle (at 61.175126 -86.685 90) (size 1.7 1.7) (drill 1) (layers "*.Cu" "*.Mask") (remove_unused_layers no)
   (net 71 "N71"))
  (pad "D10" thru_hole circle (at 63.715126 -86.685 90) (size 1.7 1.7) (drill 1) (layers "*.Cu" "*.Mask") (remove_unused_layers no)
   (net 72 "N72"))
  (pad "D10" thru_hole circle (at 64.525126 -85.225 90) (size 2 2) (drill 1.2) (layers "*.Cu" "*.Mask") (remove_unused_layers no)
   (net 72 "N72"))
  (pad "D11" thru_hole circle (at 68.725126 -85.225 90) (size 2 2) (drill 1.2) (layers "*.Cu" "*.Mask") (remove_unused_layers no)
   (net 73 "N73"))
  (pad "D11" thru_hole circle (at 69.575126 -86.685 90) (size 1.7 1.7) (drill 1) (layers "*.Cu" "*.Mask") (remove_unused_layers no)
   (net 73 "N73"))
  (pad "D12" thru_hole circle (at 72.115126 -86.685 90) (size 1.7 1.7) (drill 1) (layers "*.Cu" "*.Mask") (remove_unused_layers no)
   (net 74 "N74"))
  (pad "D12" thru_hole circle (at 72.925126 -85.225 90) (size 2 2) (drill 1.2) (layers "*.Cu" "*.Mask") (remove_unused_layers no)
   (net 74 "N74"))
  (pad "D13" thru_hole circle (at 77.125126 -85.225 90) (size 2 2) (drill 1.2) (layers "*.Cu" "*.Mask") (remove_unused_layers no)
   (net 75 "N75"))
  (pad "D13" thru_hole circle (at 77.975126 -86.685 90) (size 1.7 1.7) (drill 1) (layers "*.Cu" "*.Mask") (remove_unused_layers no)
   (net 75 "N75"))
  (pad "D14" thru_hole circle (at 80.515126 -86.685 90) (size 1.7 1.7) (drill 1) (layers "*.Cu" "*.Mask") (remove_unused_layers no)
   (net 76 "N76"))
  (pad "D14" thru_hole circle (at 81.325126 -85.225 90) (size 2 2) (drill 1.2) (layers "*.Cu" "*.Mask") (remove_unused_layers no)
   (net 76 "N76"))
  (pad "D15" thru_hole circle (at 85.525126 -85.225 90) (size 2 2) (drill 1.2) (layers "*.Cu" "*.Mask") (remove_unused_layers no)
   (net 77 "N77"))
  (pad "D15" thru_hole circle (at 86.375126 -86.685 90) (size 1.7 1.7) (drill 1) (layers "*.Cu" "*.Mask") (remove_unused_layers no)
   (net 77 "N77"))
  (pad "D16" thru_hole circle (at 88.915126 -86.685 90) (size 1.7 1.7) (drill 1) (layers "*.Cu" "*.Mask") (remove_unused_layers no)
   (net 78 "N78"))
  (pad "D16" thru_hole circle (at 89.725126 -85.225 90) (size 2 2) (drill 1.2) (layers "*.Cu" "*.Mask") (remove_unused_layers no)
   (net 78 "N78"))
  (pad "E1" thru_hole circle (at 89.290126 -78.39 180) (size 1.7 1.7) (drill 1) (layers "*.Cu" "*.Mask") (remove_unused_layers no)
   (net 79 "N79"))
  (pad "E1" thru_hole circle (at 90.750126 -79.2 90) (size 2 2) (drill 1.2) (layers "*.Cu" "*.Mask") (remove_unused_layers no)
   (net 79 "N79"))
  (pad "E2" thru_hole circle (at 89.290126 -75.85 180) (size 1.7 1.7) (drill 1) (layers "*.Cu" "*.Mask") (remove_unused_layers no)
   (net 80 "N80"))
  (pad "E2" thru_hole circle (at 90.750126 -75 90) (size 2 2) (drill 1.2) (layers "*.Cu" "*.Mask") (remove_unused_layers no) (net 80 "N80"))
  (pad "E3" thru_hole circle (at 90.750126 -70.8 90) (size 2 2) (drill 1.2) (layers "*.Cu" "*.Mask") (remove_unused_layers no)
   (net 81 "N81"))
  (pad "E4" thru_hole circle (at 85.250126 -79.2 90) (size 2 2) (drill 1.2) (layers "*.Cu" "*.Mask") (remove_unused_layers no)
   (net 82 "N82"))
  (pad "E4" thru_hole circle (at 86.750126 -78.39 180) (size 1.7 1.7) (drill 1) (layers "*.Cu" "*.Mask") (remove_unused_layers no)
   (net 82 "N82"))
  (pad "E5" thru_hole circle (at 85.250126 -75 90) (size 2 2) (drill 1.2) (layers "*.Cu" "*.Mask") (remove_unused_layers no) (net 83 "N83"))
  (pad "E5" thru_hole circle (at 86.750126 -75.85 180) (size 1.7 1.7) (drill 1) (layers "*.Cu" "*.Mask") (remove_unused_layers no)
   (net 83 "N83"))
  (pad "E6" thru_hole circle (at 85.250126 -70.8 90) (size 2 2) (drill 1.2) (layers "*.Cu" "*.Mask") (remove_unused_layers no)
   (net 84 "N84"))
  (pad "J1" thru_hole roundrect (at 83.025126 -3 90) (size 1.7 1.85) (drill 0.85) (layers "*.Cu" "*.Mask") (remove_unused_layers no)
   (roundrect_rratio 0.147059) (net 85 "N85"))
  (pad "J2" thru_hole oval (at 83.025126 -5.5 90) (size 1.7 1.85) (drill 0.85) (layers "*.Cu" "*.Mask") (remove_unused_layers no)
   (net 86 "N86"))
  (pad "J3" thru_hole oval (at 83.025126 -8 90) (size 1.7 1.85) (drill 0.85) (layers "*.Cu" "*.Mask") (remove_unused_layers no)
   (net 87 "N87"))
  (pad "J4" thru_hole oval (at 83.025126 -10.5 90) (size 1.7 1.85) (drill 0.85) (layers "*.Cu" "*.Mask") (remove_unused_layers no)
   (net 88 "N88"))
  (pad "J5" thru_hole oval (at 83.025126 -13 90) (size 1.7 1.85) (drill 0.85) (layers "*.Cu" "*.Mask") (remove_unused_layers no)
   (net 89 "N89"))
  (pad "P3" thru_hole circle (at 62.525126 -2.5) (size 1.7 1.7) (drill 1) (layers "*.Cu" "*.Mask") (remove_unused_layers no) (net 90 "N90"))
  (pad "P4" thru_hole circle (at 62.525126 -7.5) (size 1.7 1.7) (drill 1) (layers "*.Cu" "*.Mask") (remove_unused_layers no) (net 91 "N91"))
  (pad "P7" thru_hole circle (at 83.225126 -24) (size 1.7 1.7) (drill 1) (layers "*.Cu" "*.Mask") (remove_unused_layers no) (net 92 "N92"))
  (pad "P8" thru_hole circle (at 83.225126 -19.3) (size 1.7 1.7) (drill 1) (layers "*.Cu" "*.Mask") (remove_unused_layers no) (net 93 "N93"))
  (pad "P15" thru_hole circle (at 5.565126 -11.5) (size 1.7 1.7) (drill 1) (layers "*.Cu" "*.Mask") (remove_unused_layers no) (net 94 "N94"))
  (pad "P16" thru_hole circle (at 8.105126 -11.5) (size 1.7 1.7) (drill 1) (layers "*.Cu" "*.Mask") (remove_unused_layers no) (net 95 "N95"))
  (pad "P17" thru_hole circle (at 3.025126 -11.5) (size 1.7 1.7) (drill 1) (layers "*.Cu" "*.Mask") (remove_unused_layers no) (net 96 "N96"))
  (pad "P18" thru_hole circle (at 23.025126 -11) (size 1.7 1.7) (drill 1) (layers "*.Cu" "*.Mask") (remove_unused_layers no) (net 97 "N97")))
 (gr_rect (start 85 42) (end 220 147) (stroke (width 0.05) (type default)) (fill no) (layer "Edge.Cuts"))
 (segment (start 187.101 146) (end 107.5 146) (width 0.2) (layer "F.Cu") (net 2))
 (segment (start 206.5 50.04) (end 206.5 47) (width 0.2) (layer "F.Cu") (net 2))
 (segment (start 187.5 146.399) (end 187.101 146) (width 0.2) (layer "F.Cu") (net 2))
 (segment (start 189.5 146.399) (end 187.5 146.399) (width 0.2) (layer "F.Cu") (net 2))
 (segment (start 107.5 146) (end 102 140.5) (width 0.2) (layer "F.Cu") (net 2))
 (segment (start 213 122.899) (end 189.5 146.399) (width 0.2) (layer "F.Cu") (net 2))
 (segment (start 206.5 47) (end 213 47) (width 0.2) (layer "F.Cu") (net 2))
 (segment (start 213 47) (end 213 122.899) (width 0.2) (layer "F.Cu") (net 2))
 (segment (start 102 140.5) (end 102 111.587563) (width 0.2) (layer "F.Cu") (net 2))
 (segment (start 204.5 52.04) (end 206.5 50.04) (width 0.2) (layer "F.Cu") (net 2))
 (segment (start 102 111.587563) (end 103.900126 109.687437) (width 0.2) (layer "F.Cu") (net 2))
 (segment (start 96.5 80) (end 101.587563 80) (width 0.2) (layer "B.Cu") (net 3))
 (segment (start 94.5 47.5) (end 94.5 78) (width 0.2) (layer "B.Cu") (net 3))
 (segment (start 193.58 54.58) (end 187 48) (width 0.2) (layer "B.Cu") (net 3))
 (segment (start 94.5 78) (end 96.5 80) (width 0.2) (layer "B.Cu") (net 3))
 (segment (start 187 48) (end 187 47.5) (width 0.2) (layer "B.Cu") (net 3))
 (segment (start 187 47.5) (end 94.5 47.5) (width 0.2) (layer "B.Cu") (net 3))
 (segment (start 204.5 54.58) (end 193.58 54.58) (width 0.2) (layer "B.Cu") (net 3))
 (segment (start 101.587563 80) (end 103.900126 77.687437) (width 0.2) (layer "B.Cu") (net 3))
 (segment (start 111 144.5) (end 103.5 137) (width 0.2) (layer "F.Cu") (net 1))
 (segment (start 184.5 144.5) (end 111 144.5) (width 0.2) (layer "F.Cu") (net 1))
 (segment (start 187.797444 66.202556) (end 187.797444 141.202556) (width 0.2) (layer "F.Cu") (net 1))
 (segment (start 105.998996 105.487437) (end 103.900126 105.487437) (width 0.2) (layer "F.Cu") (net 1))
 (segment (start 106.5 106.011559) (end 106.511559 106) (width 0.2) (layer "F.Cu") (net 1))
 (segment (start 103.5 129) (end 106.5 126) (width 0.2) (layer "F.Cu") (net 1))
 (segment (start 106.511559 106) (end 105.998996 105.487437) (width 0.2) (layer "F.Cu") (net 1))
 (segment (start 106.5 126) (end 106.5 106.011559) (width 0.2) (layer "F.Cu") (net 1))
 (segment (start 187.797444 141.202556) (end 184.5 144.5) (width 0.2) (layer "F.Cu") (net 1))
 (segment (start 204.5 49.5) (end 187.797444 66.202556) (width 0.2) (layer "F.Cu") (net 1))
 (segment (start 103.5 137) (end 103.5 129) (width 0.2) (layer "F.Cu") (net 1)))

